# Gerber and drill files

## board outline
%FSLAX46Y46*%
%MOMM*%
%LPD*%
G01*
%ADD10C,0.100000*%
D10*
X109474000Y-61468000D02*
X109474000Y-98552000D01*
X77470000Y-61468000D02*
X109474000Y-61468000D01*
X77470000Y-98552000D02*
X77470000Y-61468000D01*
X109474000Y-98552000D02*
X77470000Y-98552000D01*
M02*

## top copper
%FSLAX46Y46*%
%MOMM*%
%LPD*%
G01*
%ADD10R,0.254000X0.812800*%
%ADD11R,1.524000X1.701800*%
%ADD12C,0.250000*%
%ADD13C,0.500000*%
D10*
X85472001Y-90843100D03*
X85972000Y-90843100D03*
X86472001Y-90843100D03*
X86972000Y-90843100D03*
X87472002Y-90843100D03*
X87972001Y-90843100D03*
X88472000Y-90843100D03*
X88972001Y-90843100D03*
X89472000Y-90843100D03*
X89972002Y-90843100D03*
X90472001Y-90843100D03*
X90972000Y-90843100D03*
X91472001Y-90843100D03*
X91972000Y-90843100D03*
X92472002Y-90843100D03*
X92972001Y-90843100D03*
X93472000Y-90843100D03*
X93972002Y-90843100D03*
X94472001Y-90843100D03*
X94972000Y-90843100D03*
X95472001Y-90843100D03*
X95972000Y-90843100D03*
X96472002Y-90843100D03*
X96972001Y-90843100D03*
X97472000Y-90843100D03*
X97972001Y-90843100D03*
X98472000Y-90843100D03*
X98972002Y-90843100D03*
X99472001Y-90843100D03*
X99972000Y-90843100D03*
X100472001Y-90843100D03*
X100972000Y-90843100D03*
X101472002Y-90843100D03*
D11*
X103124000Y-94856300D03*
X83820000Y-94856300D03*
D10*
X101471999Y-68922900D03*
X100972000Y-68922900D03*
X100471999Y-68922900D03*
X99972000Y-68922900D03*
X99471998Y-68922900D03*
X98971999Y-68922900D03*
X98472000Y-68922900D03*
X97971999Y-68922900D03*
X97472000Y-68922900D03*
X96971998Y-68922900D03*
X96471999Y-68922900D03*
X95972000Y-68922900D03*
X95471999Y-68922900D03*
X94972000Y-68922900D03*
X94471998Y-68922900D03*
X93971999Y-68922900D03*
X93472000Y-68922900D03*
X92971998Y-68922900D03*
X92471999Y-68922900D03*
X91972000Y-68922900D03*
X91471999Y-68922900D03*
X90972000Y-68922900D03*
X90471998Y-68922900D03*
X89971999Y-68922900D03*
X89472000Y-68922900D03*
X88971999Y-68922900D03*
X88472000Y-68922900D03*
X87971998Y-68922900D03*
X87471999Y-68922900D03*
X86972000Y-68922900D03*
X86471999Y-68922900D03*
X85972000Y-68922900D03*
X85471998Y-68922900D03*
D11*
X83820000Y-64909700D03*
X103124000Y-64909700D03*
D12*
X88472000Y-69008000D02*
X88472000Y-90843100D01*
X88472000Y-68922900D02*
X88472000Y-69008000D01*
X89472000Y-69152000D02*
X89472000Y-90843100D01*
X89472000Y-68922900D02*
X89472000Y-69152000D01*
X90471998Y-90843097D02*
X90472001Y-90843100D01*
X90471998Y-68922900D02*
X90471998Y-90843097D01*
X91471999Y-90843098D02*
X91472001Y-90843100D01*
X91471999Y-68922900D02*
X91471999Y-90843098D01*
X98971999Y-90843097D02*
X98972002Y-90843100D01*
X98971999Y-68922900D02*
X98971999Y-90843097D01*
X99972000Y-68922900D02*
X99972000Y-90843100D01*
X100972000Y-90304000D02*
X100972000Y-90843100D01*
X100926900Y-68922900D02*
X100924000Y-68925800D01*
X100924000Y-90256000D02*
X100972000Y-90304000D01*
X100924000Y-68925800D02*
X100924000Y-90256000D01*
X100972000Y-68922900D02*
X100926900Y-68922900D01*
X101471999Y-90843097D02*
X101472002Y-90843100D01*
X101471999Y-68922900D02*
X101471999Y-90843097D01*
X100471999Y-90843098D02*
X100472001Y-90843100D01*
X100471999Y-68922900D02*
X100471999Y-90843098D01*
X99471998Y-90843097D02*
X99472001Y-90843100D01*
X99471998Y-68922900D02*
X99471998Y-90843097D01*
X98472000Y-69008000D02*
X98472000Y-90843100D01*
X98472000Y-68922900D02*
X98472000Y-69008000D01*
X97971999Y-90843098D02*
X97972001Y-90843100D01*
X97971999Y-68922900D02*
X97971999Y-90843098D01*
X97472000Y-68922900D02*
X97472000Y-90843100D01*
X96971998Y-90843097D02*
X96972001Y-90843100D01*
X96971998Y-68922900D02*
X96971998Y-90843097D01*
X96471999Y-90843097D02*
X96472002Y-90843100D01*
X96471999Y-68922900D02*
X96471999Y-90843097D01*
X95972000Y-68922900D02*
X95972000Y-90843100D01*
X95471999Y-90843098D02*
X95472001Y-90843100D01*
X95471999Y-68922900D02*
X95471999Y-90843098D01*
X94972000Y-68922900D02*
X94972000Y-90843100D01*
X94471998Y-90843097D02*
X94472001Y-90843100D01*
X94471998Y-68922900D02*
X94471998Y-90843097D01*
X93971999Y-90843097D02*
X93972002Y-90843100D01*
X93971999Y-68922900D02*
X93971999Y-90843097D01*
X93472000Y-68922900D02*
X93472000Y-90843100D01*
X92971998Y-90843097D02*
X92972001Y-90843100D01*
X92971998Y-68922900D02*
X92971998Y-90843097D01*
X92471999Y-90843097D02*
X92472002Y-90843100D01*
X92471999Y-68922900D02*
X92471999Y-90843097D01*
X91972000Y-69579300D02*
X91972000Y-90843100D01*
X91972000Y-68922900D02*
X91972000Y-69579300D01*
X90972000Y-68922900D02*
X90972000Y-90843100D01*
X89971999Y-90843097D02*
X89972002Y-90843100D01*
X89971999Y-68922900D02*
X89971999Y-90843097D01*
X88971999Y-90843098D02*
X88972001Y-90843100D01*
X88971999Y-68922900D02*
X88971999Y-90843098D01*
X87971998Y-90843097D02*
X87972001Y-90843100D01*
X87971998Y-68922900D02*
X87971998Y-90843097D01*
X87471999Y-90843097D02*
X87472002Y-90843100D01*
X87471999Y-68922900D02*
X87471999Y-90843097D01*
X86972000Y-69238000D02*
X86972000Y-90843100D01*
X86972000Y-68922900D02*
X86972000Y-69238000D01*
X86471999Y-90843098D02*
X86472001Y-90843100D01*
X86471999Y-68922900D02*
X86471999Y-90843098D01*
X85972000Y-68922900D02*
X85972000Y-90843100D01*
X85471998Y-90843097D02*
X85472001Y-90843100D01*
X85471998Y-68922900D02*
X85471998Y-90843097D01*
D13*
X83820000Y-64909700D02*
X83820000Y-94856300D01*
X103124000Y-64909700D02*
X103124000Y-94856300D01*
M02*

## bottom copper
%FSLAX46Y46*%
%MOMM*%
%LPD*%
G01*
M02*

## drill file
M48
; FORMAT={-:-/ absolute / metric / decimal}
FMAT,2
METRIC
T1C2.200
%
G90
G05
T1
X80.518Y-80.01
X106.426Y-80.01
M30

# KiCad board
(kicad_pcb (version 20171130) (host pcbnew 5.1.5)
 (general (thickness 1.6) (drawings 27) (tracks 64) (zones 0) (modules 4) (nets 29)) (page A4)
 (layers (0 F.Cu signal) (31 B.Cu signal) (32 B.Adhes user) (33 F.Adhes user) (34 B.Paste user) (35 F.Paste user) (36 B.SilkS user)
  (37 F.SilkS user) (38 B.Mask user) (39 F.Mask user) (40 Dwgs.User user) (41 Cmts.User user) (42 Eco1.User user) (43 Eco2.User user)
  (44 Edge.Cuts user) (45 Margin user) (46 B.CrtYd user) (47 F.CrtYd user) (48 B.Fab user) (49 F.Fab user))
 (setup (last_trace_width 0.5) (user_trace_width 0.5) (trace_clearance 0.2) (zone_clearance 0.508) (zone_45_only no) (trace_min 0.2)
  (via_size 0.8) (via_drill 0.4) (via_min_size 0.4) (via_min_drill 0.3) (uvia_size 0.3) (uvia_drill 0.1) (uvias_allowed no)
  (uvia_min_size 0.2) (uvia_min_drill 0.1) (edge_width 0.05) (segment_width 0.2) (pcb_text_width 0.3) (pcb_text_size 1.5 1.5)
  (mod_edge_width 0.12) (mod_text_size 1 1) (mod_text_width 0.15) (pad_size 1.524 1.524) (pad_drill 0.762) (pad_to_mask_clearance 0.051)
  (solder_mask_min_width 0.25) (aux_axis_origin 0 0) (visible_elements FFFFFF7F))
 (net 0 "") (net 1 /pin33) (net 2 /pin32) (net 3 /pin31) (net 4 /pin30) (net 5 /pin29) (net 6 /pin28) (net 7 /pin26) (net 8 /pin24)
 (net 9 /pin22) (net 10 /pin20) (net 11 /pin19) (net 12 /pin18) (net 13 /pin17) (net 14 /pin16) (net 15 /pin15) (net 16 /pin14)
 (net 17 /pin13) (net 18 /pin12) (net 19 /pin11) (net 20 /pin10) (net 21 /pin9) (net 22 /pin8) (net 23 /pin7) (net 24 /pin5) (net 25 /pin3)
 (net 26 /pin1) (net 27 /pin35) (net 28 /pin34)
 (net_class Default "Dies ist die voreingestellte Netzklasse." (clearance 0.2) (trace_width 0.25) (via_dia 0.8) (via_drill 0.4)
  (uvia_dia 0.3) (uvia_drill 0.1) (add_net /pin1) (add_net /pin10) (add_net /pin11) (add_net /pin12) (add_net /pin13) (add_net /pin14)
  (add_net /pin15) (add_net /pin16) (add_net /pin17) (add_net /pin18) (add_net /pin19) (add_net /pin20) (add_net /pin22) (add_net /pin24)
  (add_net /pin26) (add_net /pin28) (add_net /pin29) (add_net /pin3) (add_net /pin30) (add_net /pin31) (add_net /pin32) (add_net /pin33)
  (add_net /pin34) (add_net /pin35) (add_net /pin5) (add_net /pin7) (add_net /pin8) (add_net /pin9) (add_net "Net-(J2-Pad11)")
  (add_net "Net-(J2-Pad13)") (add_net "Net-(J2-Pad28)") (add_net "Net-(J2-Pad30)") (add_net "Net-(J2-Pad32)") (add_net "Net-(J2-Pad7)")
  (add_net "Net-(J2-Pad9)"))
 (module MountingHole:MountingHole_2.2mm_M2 (layer F.Cu) (at 80.518 80.01)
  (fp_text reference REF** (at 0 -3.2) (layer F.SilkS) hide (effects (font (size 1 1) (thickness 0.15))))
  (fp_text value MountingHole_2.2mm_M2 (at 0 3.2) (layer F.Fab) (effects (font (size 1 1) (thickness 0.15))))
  (pad 1 np_thru_hole circle (at 0 0) (size 2.2 2.2) (drill 2.2) (layers *.Cu *.Mask)))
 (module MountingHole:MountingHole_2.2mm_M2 (layer F.Cu) (at 106.426 80.01)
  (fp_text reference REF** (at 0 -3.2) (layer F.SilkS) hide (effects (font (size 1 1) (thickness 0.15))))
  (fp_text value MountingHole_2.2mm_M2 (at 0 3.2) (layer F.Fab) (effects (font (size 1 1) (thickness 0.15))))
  (pad 1 np_thru_hole circle (at 0 0) (size 2.2 2.2) (drill 2.2) (layers *.Cu *.Mask)))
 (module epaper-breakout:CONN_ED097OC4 (layer F.Cu) (at 93.472 88.392 180)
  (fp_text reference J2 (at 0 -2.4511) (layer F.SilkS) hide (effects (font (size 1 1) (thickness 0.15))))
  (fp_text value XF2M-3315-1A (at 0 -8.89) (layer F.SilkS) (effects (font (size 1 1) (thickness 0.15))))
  (pad 1 smd rect (at 7.999999 -2.4511 270) (size 0.8128 0.254) (layers F.Cu F.Paste F.Mask) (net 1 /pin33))
  (pad 2 smd rect (at 7.5 -2.4511 270) (size 0.8128 0.254) (layers F.Cu F.Paste F.Mask) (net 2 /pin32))
  (pad 3 smd rect (at 6.999999 -2.4511 270) (size 0.8128 0.254) (layers F.Cu F.Paste F.Mask) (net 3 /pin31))
  (pad 4 smd rect (at 6.5 -2.4511 270) (size 0.8128 0.254) (layers F.Cu F.Paste F.Mask) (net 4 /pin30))
  (pad 5 smd rect (at 5.999998 -2.4511 270) (size 0.8128 0.254) (layers F.Cu F.Paste F.Mask) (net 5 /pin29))
  (pad 6 smd rect (at 5.499999 -2.4511 270) (size 0.8128 0.254) (layers F.Cu F.Paste F.Mask) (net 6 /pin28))
  (pad 7 smd rect (at 5 -2.4511 270) (size 0.8128 0.254) (layers F.Cu F.Paste F.Mask))
  (pad 8 smd rect (at 4.499999 -2.4511 270) (size 0.8128 0.254) (layers F.Cu F.Paste F.Mask) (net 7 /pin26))
  (pad 9 smd rect (at 4 -2.4511 270) (size 0.8128 0.254) (layers F.Cu F.Paste F.Mask))
  (pad 10 smd rect (at 3.499998 -2.4511 270) (size 0.8128 0.254) (layers F.Cu F.Paste F.Mask) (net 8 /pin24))
  (pad 11 smd rect (at 2.999999 -2.4511 270) (size 0.8128 0.254) (layers F.Cu F.Paste F.Mask))
  (pad 12 smd rect (at 2.5 -2.4511 270) (size 0.8128 0.254) (layers F.Cu F.Paste F.Mask) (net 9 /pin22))
  (pad 13 smd rect (at 1.999999 -2.4511 270) (size 0.8128 0.254) (layers F.Cu F.Paste F.Mask))
  (pad 14 smd rect (at 1.5 -2.4511 270) (size 0.8128 0.254) (layers F.Cu F.Paste F.Mask) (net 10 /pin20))
  (pad 15 smd rect (at 0.999998 -2.4511 270) (size 0.8128 0.254) (layers F.Cu F.Paste F.Mask) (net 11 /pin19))
  (pad 16 smd rect (at 0.499999 -2.4511 270) (size 0.8128 0.254) (layers F.Cu F.Paste F.Mask) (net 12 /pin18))
  (pad 17 smd rect (at 0 -2.4511 270) (size 0.8128 0.254) (layers F.Cu F.Paste F.Mask) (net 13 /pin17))
  (pad 18 smd rect (at -0.500002 -2.4511 270) (size 0.8128 0.254) (layers F.Cu F.Paste F.Mask) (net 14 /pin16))
  (pad 19 smd rect (at -1.000001 -2.4511 270) (size 0.8128 0.254) (layers F.Cu F.Paste F.Mask) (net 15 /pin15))
  (pad 20 smd rect (at -1.5 -2.4511 270) (size 0.8128 0.254) (layers F.Cu F.Paste F.Mask) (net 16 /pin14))
  (pad 21 smd rect (at -2.000001 -2.4511 270) (size 0.8128 0.254) (layers F.Cu F.Paste F.Mask) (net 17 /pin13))
  (pad 22 smd rect (at -2.5 -2.4511 270) (size 0.8128 0.254) (layers F.Cu F.Paste F.Mask) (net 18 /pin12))
  (pad 23 smd rect (at -3.000002 -2.4511 270) (size 0.8128 0.254) (layers F.Cu F.Paste F.Mask) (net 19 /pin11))
  (pad 24 smd rect (at -3.500001 -2.4511 270) (size 0.8128 0.254) (layers F.Cu F.Paste F.Mask) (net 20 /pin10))
  (pad 25 smd rect (at -4 -2.4511 270) (size 0.8128 0.254) (layers F.Cu F.Paste F.Mask) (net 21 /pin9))
  (pad 26 smd rect (at -4.500001 -2.4511 270) (size 0.8128 0.254) (layers F.Cu F.Paste F.Mask) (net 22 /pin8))
  (pad 27 smd rect (at -5 -2.4511 270) (size 0.8128 0.254) (layers F.Cu F.Paste F.Mask) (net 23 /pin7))
  (pad 28 smd rect (at -5.500002 -2.4511 270) (size 0.8128 0.254) (layers F.Cu F.Paste F.Mask))
  (pad 29 smd rect (at -6.000001 -2.4511 270) (size 0.8128 0.254) (layers F.Cu F.Paste F.Mask) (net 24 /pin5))
  (pad 30 smd rect (at -6.5 -2.4511 270) (size 0.8128 0.254) (layers F.Cu F.Paste F.Mask))
  (pad 31 smd rect (at -7.000001 -2.4511 270) (size 0.8128 0.254) (layers F.Cu F.Paste F.Mask) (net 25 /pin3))
  (pad 32 smd rect (at -7.5 -2.4511 270) (size 0.8128 0.254) (layers F.Cu F.Paste F.Mask))
  (pad 33 smd rect (at -8.000002 -2.4511 270) (size 0.8128 0.254) (layers F.Cu F.Paste F.Mask) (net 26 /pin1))
  (pad 34 smd rect (at -9.652 -6.4643 180) (size 1.524 1.7018) (layers F.Cu F.Paste F.Mask) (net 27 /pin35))
  (pad 35 smd rect (at 9.652 -6.4643 180) (size 1.524 1.7018) (layers F.Cu F.Paste F.Mask) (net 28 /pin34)))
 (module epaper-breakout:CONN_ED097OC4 (layer F.Cu) (at 93.472 71.374)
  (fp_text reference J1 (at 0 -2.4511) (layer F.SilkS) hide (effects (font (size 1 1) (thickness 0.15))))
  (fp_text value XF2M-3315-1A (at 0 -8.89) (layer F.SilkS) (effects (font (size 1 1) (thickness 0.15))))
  (pad 1 smd rect (at 7.999999 -2.4511 90) (size 0.8128 0.254) (layers F.Cu F.Paste F.Mask) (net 26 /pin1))
  (pad 2 smd rect (at 7.5 -2.4511 90) (size 0.8128 0.254) (layers F.Cu F.Paste F.Mask))
  (pad 3 smd rect (at 6.999999 -2.4511 90) (size 0.8128 0.254) (layers F.Cu F.Paste F.Mask) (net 25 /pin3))
  (pad 4 smd rect (at 6.5 -2.4511 90) (size 0.8128 0.254) (layers F.Cu F.Paste F.Mask))
  (pad 5 smd rect (at 5.999998 -2.4511 90) (size 0.8128 0.254) (layers F.Cu F.Paste F.Mask) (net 24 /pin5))
  (pad 6 smd rect (at 5.499999 -2.4511 90) (size 0.8128 0.254) (layers F.Cu F.Paste F.Mask))
  (pad 7 smd rect (at 5 -2.4511 90) (size 0.8128 0.254) (layers F.Cu F.Paste F.Mask) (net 23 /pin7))
  (pad 8 smd rect (at 4.499999 -2.4511 90) (size 0.8128 0.254) (layers F.Cu F.Paste F.Mask) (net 22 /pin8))
  (pad 9 smd rect (at 4 -2.4511 90) (size 0.8128 0.254) (layers F.Cu F.Paste F.Mask) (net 21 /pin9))
  (pad 10 smd rect (at 3.499998 -2.4511 90) (size 0.8128 0.254) (layers F.Cu F.Paste F.Mask) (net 20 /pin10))
  (pad 11 smd rect (at 2.999999 -2.4511 90) (size 0.8128 0.254) (layers F.Cu F.Paste F.Mask) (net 19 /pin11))
  (pad 12 smd rect (at 2.5 -2.4511 90) (size 0.8128 0.254) (layers F.Cu F.Paste F.Mask) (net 18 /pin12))
  (pad 13 smd rect (at 1.999999 -2.4511 90) (size 0.8128 0.254) (layers F.Cu F.Paste F.Mask) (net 17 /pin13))
  (pad 14 smd rect (at 1.5 -2.4511 90) (size 0.8128 0.254) (layers F.Cu F.Paste F.Mask) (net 16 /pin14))
  (pad 15 smd rect (at 0.999998 -2.4511 90) (size 0.8128 0.254) (layers F.Cu F.Paste F.Mask) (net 15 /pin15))
  (pad 16 smd rect (at 0.499999 -2.4511 90) (size 0.8128 0.254) (layers F.Cu F.Paste F.Mask) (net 14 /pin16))
  (pad 17 smd rect (at 0 -2.4511 90) (size 0.8128 0.254) (layers F.Cu F.Paste F.Mask) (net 13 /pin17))
  (pad 18 smd rect (at -0.500002 -2.4511 90) (size 0.8128 0.254) (layers F.Cu F.Paste F.Mask) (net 12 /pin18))
  (pad 19 smd rect (at -1.000001 -2.4511 90) (size 0.8128 0.254) (layers F.Cu F.Paste F.Mask) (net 11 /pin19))
  (pad 20 smd rect (at -1.5 -2.4511 90) (size 0.8128 0.254) (layers F.Cu F.Paste F.Mask) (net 10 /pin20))
  (pad 21 smd rect (at -2.000001 -2.4511 90) (size 0.8128 0.254) (layers F.Cu F.Paste F.Mask))
  (pad 22 smd rect (at -2.5 -2.4511 90) (size 0.8128 0.254) (layers F.Cu F.Paste F.Mask) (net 9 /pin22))
  (pad 23 smd rect (at -3.000002 -2.4511 90) (size 0.8128 0.254) (layers F.Cu F.Paste F.Mask))
  (pad 24 smd rect (at -3.500001 -2.4511 90) (size 0.8128 0.254) (layers F.Cu F.Paste F.Mask) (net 8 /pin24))
  (pad 25 smd rect (at -4 -2.4511 90) (size 0.8128 0.254) (layers F.Cu F.Paste F.Mask))
  (pad 26 smd rect (at -4.500001 -2.4511 90) (size 0.8128 0.254) (layers F.Cu F.Paste F.Mask) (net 7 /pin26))
  (pad 27 smd rect (at -5 -2.4511 90) (size 0.8128 0.254) (layers F.Cu F.Paste F.Mask))
  (pad 28 smd rect (at -5.500002 -2.4511 90) (size 0.8128 0.254) (layers F.Cu F.Paste F.Mask) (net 6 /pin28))
  (pad 29 smd rect (at -6.000001 -2.4511 90) (size 0.8128 0.254) (layers F.Cu F.Paste F.Mask) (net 5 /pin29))
  (pad 30 smd rect (at -6.5 -2.4511 90) (size 0.8128 0.254) (layers F.Cu F.Paste F.Mask) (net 4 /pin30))
  (pad 31 smd rect (at -7.000001 -2.4511 90) (size 0.8128 0.254) (layers F.Cu F.Paste F.Mask) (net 3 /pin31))
  (pad 32 smd rect (at -7.5 -2.4511 90) (size 0.8128 0.254) (layers F.Cu F.Paste F.Mask) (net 2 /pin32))
  (pad 33 smd rect (at -8.000002 -2.4511 90) (size 0.8128 0.254) (layers F.Cu F.Paste F.Mask) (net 1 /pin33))
  (pad 34 smd rect (at -9.652 -6.4643) (size 1.524 1.7018) (layers F.Cu F.Paste F.Mask) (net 28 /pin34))
  (pad 35 smd rect (at 9.652 -6.4643) (size 1.524 1.7018) (layers F.Cu F.Paste F.Mask) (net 27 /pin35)))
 (gr_line (start 109.474 61.468) (end 109.474 98.552) (layer Edge.Cuts) (width 0.1))
 (gr_line (start 77.47 61.468) (end 109.474 61.468) (layer Edge.Cuts) (width 0.1))
 (gr_line (start 77.47 98.552) (end 77.47 61.468) (layer Edge.Cuts) (width 0.1))
 (gr_line (start 109.474 98.552) (end 77.47 98.552) (layer Edge.Cuts) (width 0.1))
 (segment (start 88.472 69.008) (end 88.472 90.8431) (width 0.25) (layer F.Cu) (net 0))
 (segment (start 88.472 68.9229) (end 88.472 69.008) (width 0.25) (layer F.Cu) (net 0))
 (segment (start 89.472 69.152) (end 89.472 90.8431) (width 0.25) (layer F.Cu) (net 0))
 (segment (start 89.472 68.9229) (end 89.472 69.152) (width 0.25) (layer F.Cu) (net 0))
 (segment (start 90.471998 90.843097) (end 90.472001 90.8431) (width 0.25) (layer F.Cu) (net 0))
 (segment (start 90.471998 68.9229) (end 90.471998 90.843097) (width 0.25) (layer F.Cu) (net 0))
 (segment (start 91.471999 90.843098) (end 91.472001 90.8431) (width 0.25) (layer F.Cu) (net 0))
 (segment (start 91.471999 68.9229) (end 91.471999 90.843098) (width 0.25) (layer F.Cu) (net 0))
 (segment (start 98.971999 90.843097) (end 98.972002 90.8431) (width 0.25) (layer F.Cu) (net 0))
 (segment (start 98.971999 68.9229) (end 98.971999 90.843097) (width 0.25) (layer F.Cu) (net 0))
 (segment (start 99.972 68.9229) (end 99.972 90.8431) (width 0.25) (layer F.Cu) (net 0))
 (segment (start 100.972 90.304) (end 100.972 90.8431) (width 0.25) (layer F.Cu) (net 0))
 (segment (start 100.9269 68.9229) (end 100.924 68.9258) (width 0.25) (layer F.Cu) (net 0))
 (segment (start 100.924 90.256) (end 100.972 90.304) (width 0.25) (layer F.Cu) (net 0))
 (segment (start 100.924 68.9258) (end 100.924 90.256) (width 0.25) (layer F.Cu) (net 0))
 (segment (start 100.972 68.9229) (end 100.9269 68.9229) (width 0.25) (layer F.Cu) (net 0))
 (segment (start 101.471999 90.843097) (end 101.472002 90.8431) (width 0.25) (layer F.Cu) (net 26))
 (segment (start 101.471999 68.9229) (end 101.471999 90.843097) (width 0.25) (layer F.Cu) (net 26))
 (segment (start 100.471999 90.843098) (end 100.472001 90.8431) (width 0.25) (layer F.Cu) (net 25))
 (segment (start 100.471999 68.9229) (end 100.471999 90.843098) (width 0.25) (layer F.Cu) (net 25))
 (segment (start 99.471998 90.843097) (end 99.472001 90.8431) (width 0.25) (layer F.Cu) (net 24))
 (segment (start 99.471998 68.9229) (end 99.471998 90.843097) (width 0.25) (layer F.Cu) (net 24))
 (segment (start 98.472 69.008) (end 98.472 90.8431) (width 0.25) (layer F.Cu) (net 23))
 (segment (start 98.472 68.9229) (end 98.472 69.008) (width 0.25) (layer F.Cu) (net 23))
 (segment (start 97.971999 90.843098) (end 97.972001 90.8431) (width 0.25) (layer F.Cu) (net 22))
 (segment (start 97.971999 68.9229) (end 97.971999 90.843098) (width 0.25) (layer F.Cu) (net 22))
 (segment (start 97.472 68.9229) (end 97.472 90.8431) (width 0.25) (layer F.Cu) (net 21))
 (segment (start 96.971998 90.843097) (end 96.972001 90.8431) (width 0.25) (layer F.Cu) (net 20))
 (segment (start 96.971998 68.9229) (end 96.971998 90.843097) (width 0.25) (layer F.Cu) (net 20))
 (segment (start 96.471999 90.843097) (end 96.472002 90.8431) (width 0.25) (layer F.Cu) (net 19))
 (segment (start 96.471999 68.9229) (end 96.471999 90.843097) (width 0.25) (layer F.Cu) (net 19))
 (segment (start 95.972 68.9229) (end 95.972 90.8431) (width 0.25) (layer F.Cu) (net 18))
 (segment (start 95.471999 90.843098) (end 95.472001 90.8431) (width 0.25) (layer F.Cu) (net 17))
 (segment (start 95.471999 68.9229) (end 95.471999 90.843098) (width 0.25) (layer F.Cu) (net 17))
 (segment (start 94.972 68.9229) (end 94.972 90.8431) (width 0.25) (layer F.Cu) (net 16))
 (segment (start 94.471998 90.843097) (end 94.472001 90.8431) (width 0.25) (layer F.Cu) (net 15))
 (segment (start 94.471998 68.9229) (end 94.471998 90.843097) (width 0.25) (layer F.Cu) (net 15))
 (segment (start 93.971999 90.843097) (end 93.972002 90.8431) (width 0.25) (layer F.Cu) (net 14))
 (segment (start 93.971999 68.9229) (end 93.971999 90.843097) (width 0.25) (layer F.Cu) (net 14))
 (segment (start 93.472 68.9229) (end 93.472 90.8431) (width 0.25) (layer F.Cu) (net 13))
 (segment (start 92.971998 90.843097) (end 92.972001 90.8431) (width 0.25) (layer F.Cu) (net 12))
 (segment (start 92.971998 68.9229) (end 92.971998 90.843097) (width 0.25) (layer F.Cu) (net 12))
 (segment (start 92.471999 90.843097) (end 92.472002 90.8431) (width 0.25) (layer F.Cu) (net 11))
 (segment (start 92.471999 68.9229) (end 92.471999 90.843097) (width 0.25) (layer F.Cu) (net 11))
 (segment (start 91.972 69.5793) (end 91.972 90.8431) (width 0.25) (layer F.Cu) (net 10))
 (segment (start 91.972 68.9229) (end 91.972 69.5793) (width 0.25) (layer F.Cu) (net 10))
 (segment (start 90.972 68.9229) (end 90.972 90.8431) (width 0.25) (layer F.Cu) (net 9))
 (segment (start 89.971999 90.843097) (end 89.972002 90.8431) (width 0.25) (layer F.Cu) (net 8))
 (segment (start 89.971999 68.9229) (end 89.971999 90.843097) (width 0.25) (layer F.Cu) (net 8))
 (segment (start 88.971999 90.843098) (end 88.972001 90.8431) (width 0.25) (layer F.Cu) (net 7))
 (segment (start 88.971999 68.9229) (end 88.971999 90.843098) (width 0.25) (layer F.Cu) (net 7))
 (segment (start 87.971998 90.843097) (end 87.972001 90.8431) (width 0.25) (layer F.Cu) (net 6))
 (segment (start 87.971998 68.9229) (end 87.971998 90.843097) (width 0.25) (layer F.Cu) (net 6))
 (segment (start 87.471999 90.843097) (end 87.472002 90.8431) (width 0.25) (layer F.Cu) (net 5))
 (segment (start 87.471999 68.9229) (end 87.471999 90.843097) (width 0.25) (layer F.Cu) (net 5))
 (segment (start 86.972 69.238) (end 86.972 90.8431) (width 0.25) (layer F.Cu) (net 4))
 (segment (start 86.972 68.9229) (end 86.972 69.238) (width 0.25) (layer F.Cu) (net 4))
 (segment (start 86.471999 90.843098) (end 86.472001 90.8431) (width 0.25) (layer F.Cu) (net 3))
 (segment (start 86.471999 68.9229) (end 86.471999 90.843098) (width 0.25) (layer F.Cu) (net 3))
 (segment (start 85.972 68.9229) (end 85.972 90.8431) (width 0.25) (layer F.Cu) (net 2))
 (segment (start 85.471998 90.843097) (end 85.472001 90.8431) (width 0.25) (layer F.Cu) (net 1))
 (segment (start 85.471998 68.9229) (end 85.471998 90.843097) (width 0.25) (layer F.Cu) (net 1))
 (segment (start 83.82 64.9097) (end 83.82 94.8563) (width 0.5) (layer F.Cu) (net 28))
 (segment (start 103.124 64.9097) (end 103.124 94.8563) (width 0.5) (layer F.Cu) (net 27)))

